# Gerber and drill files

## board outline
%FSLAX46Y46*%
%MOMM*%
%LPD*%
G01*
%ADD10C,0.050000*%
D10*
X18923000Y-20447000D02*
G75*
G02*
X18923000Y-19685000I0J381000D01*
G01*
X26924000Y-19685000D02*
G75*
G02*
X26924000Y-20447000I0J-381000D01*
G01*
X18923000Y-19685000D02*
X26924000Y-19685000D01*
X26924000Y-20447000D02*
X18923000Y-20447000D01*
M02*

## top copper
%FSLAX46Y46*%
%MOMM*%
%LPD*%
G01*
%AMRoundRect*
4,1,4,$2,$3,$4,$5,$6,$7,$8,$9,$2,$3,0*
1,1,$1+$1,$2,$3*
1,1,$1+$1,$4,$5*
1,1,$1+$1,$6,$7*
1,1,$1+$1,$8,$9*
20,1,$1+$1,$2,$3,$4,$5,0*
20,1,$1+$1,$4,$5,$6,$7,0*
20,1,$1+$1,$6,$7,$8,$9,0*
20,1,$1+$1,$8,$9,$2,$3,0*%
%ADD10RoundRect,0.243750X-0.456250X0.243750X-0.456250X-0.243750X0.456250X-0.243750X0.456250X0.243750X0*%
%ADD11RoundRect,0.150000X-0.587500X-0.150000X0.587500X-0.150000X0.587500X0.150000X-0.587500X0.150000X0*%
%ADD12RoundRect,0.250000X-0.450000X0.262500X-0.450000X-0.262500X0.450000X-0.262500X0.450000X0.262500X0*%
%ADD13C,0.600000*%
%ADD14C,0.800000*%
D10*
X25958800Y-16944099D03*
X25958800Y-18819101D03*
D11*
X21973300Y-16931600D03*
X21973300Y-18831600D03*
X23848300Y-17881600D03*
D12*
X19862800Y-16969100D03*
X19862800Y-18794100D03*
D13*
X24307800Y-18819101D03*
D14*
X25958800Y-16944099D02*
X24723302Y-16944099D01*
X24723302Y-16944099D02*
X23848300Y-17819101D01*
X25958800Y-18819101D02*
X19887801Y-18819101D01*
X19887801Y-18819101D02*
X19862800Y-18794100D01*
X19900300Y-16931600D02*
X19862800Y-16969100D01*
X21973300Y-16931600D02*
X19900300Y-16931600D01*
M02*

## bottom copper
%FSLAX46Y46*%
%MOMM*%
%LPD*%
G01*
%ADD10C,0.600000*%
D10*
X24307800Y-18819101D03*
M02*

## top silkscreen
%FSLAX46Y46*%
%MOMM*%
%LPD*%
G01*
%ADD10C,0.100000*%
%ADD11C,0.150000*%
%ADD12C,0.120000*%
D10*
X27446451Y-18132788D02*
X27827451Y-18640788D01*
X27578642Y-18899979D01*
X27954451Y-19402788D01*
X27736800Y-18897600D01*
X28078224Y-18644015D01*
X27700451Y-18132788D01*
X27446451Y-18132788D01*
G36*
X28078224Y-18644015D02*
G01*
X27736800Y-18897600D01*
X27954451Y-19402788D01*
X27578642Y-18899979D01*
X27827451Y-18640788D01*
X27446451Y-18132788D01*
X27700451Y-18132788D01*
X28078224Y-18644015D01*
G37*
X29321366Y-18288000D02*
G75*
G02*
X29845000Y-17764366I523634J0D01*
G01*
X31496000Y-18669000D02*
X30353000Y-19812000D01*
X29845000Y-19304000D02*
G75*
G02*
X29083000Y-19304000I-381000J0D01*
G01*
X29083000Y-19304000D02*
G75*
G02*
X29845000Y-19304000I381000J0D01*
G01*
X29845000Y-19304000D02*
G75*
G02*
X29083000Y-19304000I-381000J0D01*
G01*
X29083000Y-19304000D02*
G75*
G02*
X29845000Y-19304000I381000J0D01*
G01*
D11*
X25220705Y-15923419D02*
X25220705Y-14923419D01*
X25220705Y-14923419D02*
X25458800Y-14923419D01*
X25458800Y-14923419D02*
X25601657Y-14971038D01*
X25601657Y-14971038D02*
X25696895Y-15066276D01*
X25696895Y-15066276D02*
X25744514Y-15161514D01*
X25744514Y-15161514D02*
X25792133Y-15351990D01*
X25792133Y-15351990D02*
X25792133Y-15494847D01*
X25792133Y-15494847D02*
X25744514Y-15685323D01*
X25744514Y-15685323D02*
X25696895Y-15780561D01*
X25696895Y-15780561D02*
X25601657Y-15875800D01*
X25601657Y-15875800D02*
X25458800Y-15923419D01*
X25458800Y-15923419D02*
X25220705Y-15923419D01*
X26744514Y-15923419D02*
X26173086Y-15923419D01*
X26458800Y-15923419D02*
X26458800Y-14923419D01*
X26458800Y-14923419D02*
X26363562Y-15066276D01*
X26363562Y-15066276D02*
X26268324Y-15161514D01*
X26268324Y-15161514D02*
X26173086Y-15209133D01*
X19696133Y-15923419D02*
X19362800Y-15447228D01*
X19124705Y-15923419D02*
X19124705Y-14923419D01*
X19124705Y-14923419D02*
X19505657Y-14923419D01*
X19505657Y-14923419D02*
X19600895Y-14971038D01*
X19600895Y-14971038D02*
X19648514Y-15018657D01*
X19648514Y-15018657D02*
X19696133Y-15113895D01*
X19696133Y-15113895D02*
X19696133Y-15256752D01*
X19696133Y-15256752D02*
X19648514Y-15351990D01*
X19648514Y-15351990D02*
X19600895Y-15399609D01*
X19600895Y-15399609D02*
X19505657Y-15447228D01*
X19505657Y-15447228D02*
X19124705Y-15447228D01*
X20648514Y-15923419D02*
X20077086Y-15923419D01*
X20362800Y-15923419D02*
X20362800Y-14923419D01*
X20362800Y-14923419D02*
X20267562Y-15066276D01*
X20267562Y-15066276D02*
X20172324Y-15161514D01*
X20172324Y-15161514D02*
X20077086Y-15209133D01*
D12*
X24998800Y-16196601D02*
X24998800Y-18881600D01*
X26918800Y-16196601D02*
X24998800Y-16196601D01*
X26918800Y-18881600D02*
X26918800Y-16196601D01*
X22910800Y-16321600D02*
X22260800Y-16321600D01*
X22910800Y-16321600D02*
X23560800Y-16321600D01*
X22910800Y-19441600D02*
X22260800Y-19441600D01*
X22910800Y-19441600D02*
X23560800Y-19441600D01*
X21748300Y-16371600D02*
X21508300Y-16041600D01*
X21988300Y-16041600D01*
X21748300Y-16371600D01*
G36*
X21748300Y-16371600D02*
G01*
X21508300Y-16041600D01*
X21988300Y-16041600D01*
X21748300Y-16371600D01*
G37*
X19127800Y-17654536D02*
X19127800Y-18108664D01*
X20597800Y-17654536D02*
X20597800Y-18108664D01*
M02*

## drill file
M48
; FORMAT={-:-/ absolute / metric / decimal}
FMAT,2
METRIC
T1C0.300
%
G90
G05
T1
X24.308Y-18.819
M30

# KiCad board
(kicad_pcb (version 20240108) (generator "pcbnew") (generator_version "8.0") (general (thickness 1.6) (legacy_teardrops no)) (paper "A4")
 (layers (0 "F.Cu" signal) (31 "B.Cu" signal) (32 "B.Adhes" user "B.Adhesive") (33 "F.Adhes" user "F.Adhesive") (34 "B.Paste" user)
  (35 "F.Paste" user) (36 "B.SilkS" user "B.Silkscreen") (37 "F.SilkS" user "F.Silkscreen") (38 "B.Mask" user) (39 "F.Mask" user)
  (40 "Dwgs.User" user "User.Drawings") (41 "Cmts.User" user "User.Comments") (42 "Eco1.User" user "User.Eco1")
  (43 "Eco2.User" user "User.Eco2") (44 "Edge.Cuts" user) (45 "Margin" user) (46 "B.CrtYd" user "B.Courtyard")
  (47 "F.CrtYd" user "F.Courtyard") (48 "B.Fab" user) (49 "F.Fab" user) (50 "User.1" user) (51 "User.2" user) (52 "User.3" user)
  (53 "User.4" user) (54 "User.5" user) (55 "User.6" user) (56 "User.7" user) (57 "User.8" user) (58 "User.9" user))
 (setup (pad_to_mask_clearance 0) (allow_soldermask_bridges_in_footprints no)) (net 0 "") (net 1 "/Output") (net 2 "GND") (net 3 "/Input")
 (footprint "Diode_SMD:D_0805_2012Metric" (layer "F.Cu") (at 25.9588 17.8816 -90)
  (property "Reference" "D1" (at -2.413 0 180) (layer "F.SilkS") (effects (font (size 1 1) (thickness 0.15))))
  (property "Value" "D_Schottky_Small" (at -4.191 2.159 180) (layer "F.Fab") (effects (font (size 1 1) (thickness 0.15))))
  (fp_line (start -1.684999 0.96) (end 1 0.96) (stroke (width 0.12) (type solid)) (layer "F.SilkS"))
  (fp_line (start -1.684999 -0.96) (end -1.684999 0.96) (stroke (width 0.12) (type solid)) (layer "F.SilkS"))
  (fp_line (start 1 -0.96) (end -1.684999 -0.96) (stroke (width 0.12) (type solid)) (layer "F.SilkS"))
  (pad "1" smd roundrect (at -0.937501 0 270) (size 0.975 1.4) (layers "F.Cu" "F.Paste" "F.Mask") (roundrect_rratio 0.25) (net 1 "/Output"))
  (pad "2" smd roundrect (at 0.937501 0 270) (size 0.975 1.4) (layers "F.Cu" "F.Paste" "F.Mask") (roundrect_rratio 0.25) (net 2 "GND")))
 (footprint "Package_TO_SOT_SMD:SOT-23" (layer "F.Cu") (at 22.9108 17.8816)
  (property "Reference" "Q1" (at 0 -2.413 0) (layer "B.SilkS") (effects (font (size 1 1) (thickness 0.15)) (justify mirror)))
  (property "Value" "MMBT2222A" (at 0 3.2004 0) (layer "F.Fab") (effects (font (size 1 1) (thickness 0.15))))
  (fp_line (start 0 -1.56) (end -0.65 -1.56) (stroke (width 0.12) (type solid)) (layer "F.SilkS"))
  (fp_line (start 0 -1.56) (end 0.65 -1.56) (stroke (width 0.12) (type solid)) (layer "F.SilkS"))
  (fp_line (start 0 1.56) (end -0.65 1.56) (stroke (width 0.12) (type solid)) (layer "F.SilkS"))
  (fp_line (start 0 1.56) (end 0.65 1.56) (stroke (width 0.12) (type solid)) (layer "F.SilkS"))
  (fp_poly
   (pts (xy -1.1625 -1.51) (xy -1.4025 -1.84) (xy -0.9225 -1.84) (xy -1.1625 -1.51)) (stroke (width 0.12) (type solid)) (fill solid)
   (layer "F.SilkS"))
  (pad "1" smd roundrect (at -0.9375 -0.95) (size 1.475 0.6) (layers "F.Cu" "F.Paste" "F.Mask") (roundrect_rratio 0.25) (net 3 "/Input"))
  (pad "2" smd roundrect (at -0.9375 0.95) (size 1.475 0.6) (layers "F.Cu" "F.Paste" "F.Mask") (roundrect_rratio 0.25) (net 2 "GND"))
  (pad "3" smd roundrect (at 0.9375 0) (size 1.475 0.6) (layers "F.Cu" "F.Paste" "F.Mask") (roundrect_rratio 0.25) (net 1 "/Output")))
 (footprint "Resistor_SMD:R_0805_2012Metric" (layer "F.Cu") (at 19.8628 17.8816 -90)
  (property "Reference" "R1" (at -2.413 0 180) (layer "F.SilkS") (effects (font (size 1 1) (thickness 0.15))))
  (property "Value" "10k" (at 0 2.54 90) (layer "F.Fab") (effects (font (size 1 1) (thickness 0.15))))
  (fp_line (start -0.227064 0.735) (end 0.227064 0.735) (stroke (width 0.12) (type solid)) (layer "F.SilkS"))
  (fp_line (start -0.227064 -0.735) (end 0.227064 -0.735) (stroke (width 0.12) (type solid)) (layer "F.SilkS"))
  (pad "1" smd roundrect (at -0.9125 0 270) (size 1.025 1.4) (layers "F.Cu" "F.Paste" "F.Mask") (roundrect_rratio 0.243902) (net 3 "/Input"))
  (pad "2" smd roundrect (at 0.9125 0 270) (size 1.025 1.4) (layers "F.Cu" "F.Paste" "F.Mask") (roundrect_rratio 0.243902) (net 2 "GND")))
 (gr_poly
  (pts (xy 27.446451 18.132788) (xy 27.827451 18.640788) (xy 27.578642 18.899979) (xy 27.954451 19.402788) (xy 27.7368 18.8976)
   (xy 28.078224 18.644015) (xy 27.700451 18.132788))
  (stroke (width 0.1) (type solid)) (fill solid) (layer "F.SilkS"))
 (gr_arc (start 29.321366 18.288) (mid 29.474735 17.917735) (end 29.845 17.764366) (stroke (width 0.1) (type default)) (layer "F.SilkS"))
 (gr_line (start 31.496 18.669) (end 30.353 19.812) (stroke (width 0.1) (type default)) (layer "F.SilkS"))
 (gr_circle (center 29.464 19.304) (end 29.464 18.923) (stroke (width 0.1) (type default)) (fill none) (layer "F.SilkS"))
 (gr_circle (center 29.464 19.304) (end 29.464 18.923) (stroke (width 0.1) (type default)) (fill none) (layer "F.SilkS"))
 (gr_arc (start 18.923 20.447) (mid 18.542 20.066) (end 18.923 19.685) (stroke (width 0.05) (type default)) (layer "Edge.Cuts"))
 (gr_arc (start 26.924 19.685) (mid 27.305 20.066) (end 26.924 20.447) (stroke (width 0.05) (type default)) (layer "Edge.Cuts"))
 (gr_line (start 18.923 19.685) (end 26.924 19.685) (stroke (width 0.05) (type default)) (layer "Edge.Cuts"))
 (gr_line (start 26.924 20.447) (end 18.923 20.447) (stroke (width 0.05) (type default)) (layer "Edge.Cuts"))
 (segment (start 25.9588 16.944099) (end 24.723302 16.944099) (width 0.8) (layer "F.Cu") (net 1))
 (segment (start 24.723302 16.944099) (end 23.8483 17.819101) (width 0.8) (layer "F.Cu") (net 1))
 (segment (start 25.9588 18.819101) (end 19.887801 18.819101) (width 0.8) (layer "F.Cu") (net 2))
 (segment (start 19.887801 18.819101) (end 19.8628 18.7941) (width 0.8) (layer "F.Cu") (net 2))
 (via (at 24.3078 18.819101) (size 0.6) (drill 0.3) (layers "F.Cu" "B.Cu") (free yes) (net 2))
 (segment (start 19.9003 16.9316) (end 19.8628 16.9691) (width 0.8) (layer "F.Cu") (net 3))
 (segment (start 21.9733 16.9316) (end 19.9003 16.9316) (width 0.8) (layer "F.Cu") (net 3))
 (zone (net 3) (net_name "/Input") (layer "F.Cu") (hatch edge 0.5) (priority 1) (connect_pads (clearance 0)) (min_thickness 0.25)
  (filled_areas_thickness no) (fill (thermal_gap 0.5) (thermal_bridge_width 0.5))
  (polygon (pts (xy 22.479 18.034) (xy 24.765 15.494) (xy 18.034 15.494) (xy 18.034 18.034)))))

